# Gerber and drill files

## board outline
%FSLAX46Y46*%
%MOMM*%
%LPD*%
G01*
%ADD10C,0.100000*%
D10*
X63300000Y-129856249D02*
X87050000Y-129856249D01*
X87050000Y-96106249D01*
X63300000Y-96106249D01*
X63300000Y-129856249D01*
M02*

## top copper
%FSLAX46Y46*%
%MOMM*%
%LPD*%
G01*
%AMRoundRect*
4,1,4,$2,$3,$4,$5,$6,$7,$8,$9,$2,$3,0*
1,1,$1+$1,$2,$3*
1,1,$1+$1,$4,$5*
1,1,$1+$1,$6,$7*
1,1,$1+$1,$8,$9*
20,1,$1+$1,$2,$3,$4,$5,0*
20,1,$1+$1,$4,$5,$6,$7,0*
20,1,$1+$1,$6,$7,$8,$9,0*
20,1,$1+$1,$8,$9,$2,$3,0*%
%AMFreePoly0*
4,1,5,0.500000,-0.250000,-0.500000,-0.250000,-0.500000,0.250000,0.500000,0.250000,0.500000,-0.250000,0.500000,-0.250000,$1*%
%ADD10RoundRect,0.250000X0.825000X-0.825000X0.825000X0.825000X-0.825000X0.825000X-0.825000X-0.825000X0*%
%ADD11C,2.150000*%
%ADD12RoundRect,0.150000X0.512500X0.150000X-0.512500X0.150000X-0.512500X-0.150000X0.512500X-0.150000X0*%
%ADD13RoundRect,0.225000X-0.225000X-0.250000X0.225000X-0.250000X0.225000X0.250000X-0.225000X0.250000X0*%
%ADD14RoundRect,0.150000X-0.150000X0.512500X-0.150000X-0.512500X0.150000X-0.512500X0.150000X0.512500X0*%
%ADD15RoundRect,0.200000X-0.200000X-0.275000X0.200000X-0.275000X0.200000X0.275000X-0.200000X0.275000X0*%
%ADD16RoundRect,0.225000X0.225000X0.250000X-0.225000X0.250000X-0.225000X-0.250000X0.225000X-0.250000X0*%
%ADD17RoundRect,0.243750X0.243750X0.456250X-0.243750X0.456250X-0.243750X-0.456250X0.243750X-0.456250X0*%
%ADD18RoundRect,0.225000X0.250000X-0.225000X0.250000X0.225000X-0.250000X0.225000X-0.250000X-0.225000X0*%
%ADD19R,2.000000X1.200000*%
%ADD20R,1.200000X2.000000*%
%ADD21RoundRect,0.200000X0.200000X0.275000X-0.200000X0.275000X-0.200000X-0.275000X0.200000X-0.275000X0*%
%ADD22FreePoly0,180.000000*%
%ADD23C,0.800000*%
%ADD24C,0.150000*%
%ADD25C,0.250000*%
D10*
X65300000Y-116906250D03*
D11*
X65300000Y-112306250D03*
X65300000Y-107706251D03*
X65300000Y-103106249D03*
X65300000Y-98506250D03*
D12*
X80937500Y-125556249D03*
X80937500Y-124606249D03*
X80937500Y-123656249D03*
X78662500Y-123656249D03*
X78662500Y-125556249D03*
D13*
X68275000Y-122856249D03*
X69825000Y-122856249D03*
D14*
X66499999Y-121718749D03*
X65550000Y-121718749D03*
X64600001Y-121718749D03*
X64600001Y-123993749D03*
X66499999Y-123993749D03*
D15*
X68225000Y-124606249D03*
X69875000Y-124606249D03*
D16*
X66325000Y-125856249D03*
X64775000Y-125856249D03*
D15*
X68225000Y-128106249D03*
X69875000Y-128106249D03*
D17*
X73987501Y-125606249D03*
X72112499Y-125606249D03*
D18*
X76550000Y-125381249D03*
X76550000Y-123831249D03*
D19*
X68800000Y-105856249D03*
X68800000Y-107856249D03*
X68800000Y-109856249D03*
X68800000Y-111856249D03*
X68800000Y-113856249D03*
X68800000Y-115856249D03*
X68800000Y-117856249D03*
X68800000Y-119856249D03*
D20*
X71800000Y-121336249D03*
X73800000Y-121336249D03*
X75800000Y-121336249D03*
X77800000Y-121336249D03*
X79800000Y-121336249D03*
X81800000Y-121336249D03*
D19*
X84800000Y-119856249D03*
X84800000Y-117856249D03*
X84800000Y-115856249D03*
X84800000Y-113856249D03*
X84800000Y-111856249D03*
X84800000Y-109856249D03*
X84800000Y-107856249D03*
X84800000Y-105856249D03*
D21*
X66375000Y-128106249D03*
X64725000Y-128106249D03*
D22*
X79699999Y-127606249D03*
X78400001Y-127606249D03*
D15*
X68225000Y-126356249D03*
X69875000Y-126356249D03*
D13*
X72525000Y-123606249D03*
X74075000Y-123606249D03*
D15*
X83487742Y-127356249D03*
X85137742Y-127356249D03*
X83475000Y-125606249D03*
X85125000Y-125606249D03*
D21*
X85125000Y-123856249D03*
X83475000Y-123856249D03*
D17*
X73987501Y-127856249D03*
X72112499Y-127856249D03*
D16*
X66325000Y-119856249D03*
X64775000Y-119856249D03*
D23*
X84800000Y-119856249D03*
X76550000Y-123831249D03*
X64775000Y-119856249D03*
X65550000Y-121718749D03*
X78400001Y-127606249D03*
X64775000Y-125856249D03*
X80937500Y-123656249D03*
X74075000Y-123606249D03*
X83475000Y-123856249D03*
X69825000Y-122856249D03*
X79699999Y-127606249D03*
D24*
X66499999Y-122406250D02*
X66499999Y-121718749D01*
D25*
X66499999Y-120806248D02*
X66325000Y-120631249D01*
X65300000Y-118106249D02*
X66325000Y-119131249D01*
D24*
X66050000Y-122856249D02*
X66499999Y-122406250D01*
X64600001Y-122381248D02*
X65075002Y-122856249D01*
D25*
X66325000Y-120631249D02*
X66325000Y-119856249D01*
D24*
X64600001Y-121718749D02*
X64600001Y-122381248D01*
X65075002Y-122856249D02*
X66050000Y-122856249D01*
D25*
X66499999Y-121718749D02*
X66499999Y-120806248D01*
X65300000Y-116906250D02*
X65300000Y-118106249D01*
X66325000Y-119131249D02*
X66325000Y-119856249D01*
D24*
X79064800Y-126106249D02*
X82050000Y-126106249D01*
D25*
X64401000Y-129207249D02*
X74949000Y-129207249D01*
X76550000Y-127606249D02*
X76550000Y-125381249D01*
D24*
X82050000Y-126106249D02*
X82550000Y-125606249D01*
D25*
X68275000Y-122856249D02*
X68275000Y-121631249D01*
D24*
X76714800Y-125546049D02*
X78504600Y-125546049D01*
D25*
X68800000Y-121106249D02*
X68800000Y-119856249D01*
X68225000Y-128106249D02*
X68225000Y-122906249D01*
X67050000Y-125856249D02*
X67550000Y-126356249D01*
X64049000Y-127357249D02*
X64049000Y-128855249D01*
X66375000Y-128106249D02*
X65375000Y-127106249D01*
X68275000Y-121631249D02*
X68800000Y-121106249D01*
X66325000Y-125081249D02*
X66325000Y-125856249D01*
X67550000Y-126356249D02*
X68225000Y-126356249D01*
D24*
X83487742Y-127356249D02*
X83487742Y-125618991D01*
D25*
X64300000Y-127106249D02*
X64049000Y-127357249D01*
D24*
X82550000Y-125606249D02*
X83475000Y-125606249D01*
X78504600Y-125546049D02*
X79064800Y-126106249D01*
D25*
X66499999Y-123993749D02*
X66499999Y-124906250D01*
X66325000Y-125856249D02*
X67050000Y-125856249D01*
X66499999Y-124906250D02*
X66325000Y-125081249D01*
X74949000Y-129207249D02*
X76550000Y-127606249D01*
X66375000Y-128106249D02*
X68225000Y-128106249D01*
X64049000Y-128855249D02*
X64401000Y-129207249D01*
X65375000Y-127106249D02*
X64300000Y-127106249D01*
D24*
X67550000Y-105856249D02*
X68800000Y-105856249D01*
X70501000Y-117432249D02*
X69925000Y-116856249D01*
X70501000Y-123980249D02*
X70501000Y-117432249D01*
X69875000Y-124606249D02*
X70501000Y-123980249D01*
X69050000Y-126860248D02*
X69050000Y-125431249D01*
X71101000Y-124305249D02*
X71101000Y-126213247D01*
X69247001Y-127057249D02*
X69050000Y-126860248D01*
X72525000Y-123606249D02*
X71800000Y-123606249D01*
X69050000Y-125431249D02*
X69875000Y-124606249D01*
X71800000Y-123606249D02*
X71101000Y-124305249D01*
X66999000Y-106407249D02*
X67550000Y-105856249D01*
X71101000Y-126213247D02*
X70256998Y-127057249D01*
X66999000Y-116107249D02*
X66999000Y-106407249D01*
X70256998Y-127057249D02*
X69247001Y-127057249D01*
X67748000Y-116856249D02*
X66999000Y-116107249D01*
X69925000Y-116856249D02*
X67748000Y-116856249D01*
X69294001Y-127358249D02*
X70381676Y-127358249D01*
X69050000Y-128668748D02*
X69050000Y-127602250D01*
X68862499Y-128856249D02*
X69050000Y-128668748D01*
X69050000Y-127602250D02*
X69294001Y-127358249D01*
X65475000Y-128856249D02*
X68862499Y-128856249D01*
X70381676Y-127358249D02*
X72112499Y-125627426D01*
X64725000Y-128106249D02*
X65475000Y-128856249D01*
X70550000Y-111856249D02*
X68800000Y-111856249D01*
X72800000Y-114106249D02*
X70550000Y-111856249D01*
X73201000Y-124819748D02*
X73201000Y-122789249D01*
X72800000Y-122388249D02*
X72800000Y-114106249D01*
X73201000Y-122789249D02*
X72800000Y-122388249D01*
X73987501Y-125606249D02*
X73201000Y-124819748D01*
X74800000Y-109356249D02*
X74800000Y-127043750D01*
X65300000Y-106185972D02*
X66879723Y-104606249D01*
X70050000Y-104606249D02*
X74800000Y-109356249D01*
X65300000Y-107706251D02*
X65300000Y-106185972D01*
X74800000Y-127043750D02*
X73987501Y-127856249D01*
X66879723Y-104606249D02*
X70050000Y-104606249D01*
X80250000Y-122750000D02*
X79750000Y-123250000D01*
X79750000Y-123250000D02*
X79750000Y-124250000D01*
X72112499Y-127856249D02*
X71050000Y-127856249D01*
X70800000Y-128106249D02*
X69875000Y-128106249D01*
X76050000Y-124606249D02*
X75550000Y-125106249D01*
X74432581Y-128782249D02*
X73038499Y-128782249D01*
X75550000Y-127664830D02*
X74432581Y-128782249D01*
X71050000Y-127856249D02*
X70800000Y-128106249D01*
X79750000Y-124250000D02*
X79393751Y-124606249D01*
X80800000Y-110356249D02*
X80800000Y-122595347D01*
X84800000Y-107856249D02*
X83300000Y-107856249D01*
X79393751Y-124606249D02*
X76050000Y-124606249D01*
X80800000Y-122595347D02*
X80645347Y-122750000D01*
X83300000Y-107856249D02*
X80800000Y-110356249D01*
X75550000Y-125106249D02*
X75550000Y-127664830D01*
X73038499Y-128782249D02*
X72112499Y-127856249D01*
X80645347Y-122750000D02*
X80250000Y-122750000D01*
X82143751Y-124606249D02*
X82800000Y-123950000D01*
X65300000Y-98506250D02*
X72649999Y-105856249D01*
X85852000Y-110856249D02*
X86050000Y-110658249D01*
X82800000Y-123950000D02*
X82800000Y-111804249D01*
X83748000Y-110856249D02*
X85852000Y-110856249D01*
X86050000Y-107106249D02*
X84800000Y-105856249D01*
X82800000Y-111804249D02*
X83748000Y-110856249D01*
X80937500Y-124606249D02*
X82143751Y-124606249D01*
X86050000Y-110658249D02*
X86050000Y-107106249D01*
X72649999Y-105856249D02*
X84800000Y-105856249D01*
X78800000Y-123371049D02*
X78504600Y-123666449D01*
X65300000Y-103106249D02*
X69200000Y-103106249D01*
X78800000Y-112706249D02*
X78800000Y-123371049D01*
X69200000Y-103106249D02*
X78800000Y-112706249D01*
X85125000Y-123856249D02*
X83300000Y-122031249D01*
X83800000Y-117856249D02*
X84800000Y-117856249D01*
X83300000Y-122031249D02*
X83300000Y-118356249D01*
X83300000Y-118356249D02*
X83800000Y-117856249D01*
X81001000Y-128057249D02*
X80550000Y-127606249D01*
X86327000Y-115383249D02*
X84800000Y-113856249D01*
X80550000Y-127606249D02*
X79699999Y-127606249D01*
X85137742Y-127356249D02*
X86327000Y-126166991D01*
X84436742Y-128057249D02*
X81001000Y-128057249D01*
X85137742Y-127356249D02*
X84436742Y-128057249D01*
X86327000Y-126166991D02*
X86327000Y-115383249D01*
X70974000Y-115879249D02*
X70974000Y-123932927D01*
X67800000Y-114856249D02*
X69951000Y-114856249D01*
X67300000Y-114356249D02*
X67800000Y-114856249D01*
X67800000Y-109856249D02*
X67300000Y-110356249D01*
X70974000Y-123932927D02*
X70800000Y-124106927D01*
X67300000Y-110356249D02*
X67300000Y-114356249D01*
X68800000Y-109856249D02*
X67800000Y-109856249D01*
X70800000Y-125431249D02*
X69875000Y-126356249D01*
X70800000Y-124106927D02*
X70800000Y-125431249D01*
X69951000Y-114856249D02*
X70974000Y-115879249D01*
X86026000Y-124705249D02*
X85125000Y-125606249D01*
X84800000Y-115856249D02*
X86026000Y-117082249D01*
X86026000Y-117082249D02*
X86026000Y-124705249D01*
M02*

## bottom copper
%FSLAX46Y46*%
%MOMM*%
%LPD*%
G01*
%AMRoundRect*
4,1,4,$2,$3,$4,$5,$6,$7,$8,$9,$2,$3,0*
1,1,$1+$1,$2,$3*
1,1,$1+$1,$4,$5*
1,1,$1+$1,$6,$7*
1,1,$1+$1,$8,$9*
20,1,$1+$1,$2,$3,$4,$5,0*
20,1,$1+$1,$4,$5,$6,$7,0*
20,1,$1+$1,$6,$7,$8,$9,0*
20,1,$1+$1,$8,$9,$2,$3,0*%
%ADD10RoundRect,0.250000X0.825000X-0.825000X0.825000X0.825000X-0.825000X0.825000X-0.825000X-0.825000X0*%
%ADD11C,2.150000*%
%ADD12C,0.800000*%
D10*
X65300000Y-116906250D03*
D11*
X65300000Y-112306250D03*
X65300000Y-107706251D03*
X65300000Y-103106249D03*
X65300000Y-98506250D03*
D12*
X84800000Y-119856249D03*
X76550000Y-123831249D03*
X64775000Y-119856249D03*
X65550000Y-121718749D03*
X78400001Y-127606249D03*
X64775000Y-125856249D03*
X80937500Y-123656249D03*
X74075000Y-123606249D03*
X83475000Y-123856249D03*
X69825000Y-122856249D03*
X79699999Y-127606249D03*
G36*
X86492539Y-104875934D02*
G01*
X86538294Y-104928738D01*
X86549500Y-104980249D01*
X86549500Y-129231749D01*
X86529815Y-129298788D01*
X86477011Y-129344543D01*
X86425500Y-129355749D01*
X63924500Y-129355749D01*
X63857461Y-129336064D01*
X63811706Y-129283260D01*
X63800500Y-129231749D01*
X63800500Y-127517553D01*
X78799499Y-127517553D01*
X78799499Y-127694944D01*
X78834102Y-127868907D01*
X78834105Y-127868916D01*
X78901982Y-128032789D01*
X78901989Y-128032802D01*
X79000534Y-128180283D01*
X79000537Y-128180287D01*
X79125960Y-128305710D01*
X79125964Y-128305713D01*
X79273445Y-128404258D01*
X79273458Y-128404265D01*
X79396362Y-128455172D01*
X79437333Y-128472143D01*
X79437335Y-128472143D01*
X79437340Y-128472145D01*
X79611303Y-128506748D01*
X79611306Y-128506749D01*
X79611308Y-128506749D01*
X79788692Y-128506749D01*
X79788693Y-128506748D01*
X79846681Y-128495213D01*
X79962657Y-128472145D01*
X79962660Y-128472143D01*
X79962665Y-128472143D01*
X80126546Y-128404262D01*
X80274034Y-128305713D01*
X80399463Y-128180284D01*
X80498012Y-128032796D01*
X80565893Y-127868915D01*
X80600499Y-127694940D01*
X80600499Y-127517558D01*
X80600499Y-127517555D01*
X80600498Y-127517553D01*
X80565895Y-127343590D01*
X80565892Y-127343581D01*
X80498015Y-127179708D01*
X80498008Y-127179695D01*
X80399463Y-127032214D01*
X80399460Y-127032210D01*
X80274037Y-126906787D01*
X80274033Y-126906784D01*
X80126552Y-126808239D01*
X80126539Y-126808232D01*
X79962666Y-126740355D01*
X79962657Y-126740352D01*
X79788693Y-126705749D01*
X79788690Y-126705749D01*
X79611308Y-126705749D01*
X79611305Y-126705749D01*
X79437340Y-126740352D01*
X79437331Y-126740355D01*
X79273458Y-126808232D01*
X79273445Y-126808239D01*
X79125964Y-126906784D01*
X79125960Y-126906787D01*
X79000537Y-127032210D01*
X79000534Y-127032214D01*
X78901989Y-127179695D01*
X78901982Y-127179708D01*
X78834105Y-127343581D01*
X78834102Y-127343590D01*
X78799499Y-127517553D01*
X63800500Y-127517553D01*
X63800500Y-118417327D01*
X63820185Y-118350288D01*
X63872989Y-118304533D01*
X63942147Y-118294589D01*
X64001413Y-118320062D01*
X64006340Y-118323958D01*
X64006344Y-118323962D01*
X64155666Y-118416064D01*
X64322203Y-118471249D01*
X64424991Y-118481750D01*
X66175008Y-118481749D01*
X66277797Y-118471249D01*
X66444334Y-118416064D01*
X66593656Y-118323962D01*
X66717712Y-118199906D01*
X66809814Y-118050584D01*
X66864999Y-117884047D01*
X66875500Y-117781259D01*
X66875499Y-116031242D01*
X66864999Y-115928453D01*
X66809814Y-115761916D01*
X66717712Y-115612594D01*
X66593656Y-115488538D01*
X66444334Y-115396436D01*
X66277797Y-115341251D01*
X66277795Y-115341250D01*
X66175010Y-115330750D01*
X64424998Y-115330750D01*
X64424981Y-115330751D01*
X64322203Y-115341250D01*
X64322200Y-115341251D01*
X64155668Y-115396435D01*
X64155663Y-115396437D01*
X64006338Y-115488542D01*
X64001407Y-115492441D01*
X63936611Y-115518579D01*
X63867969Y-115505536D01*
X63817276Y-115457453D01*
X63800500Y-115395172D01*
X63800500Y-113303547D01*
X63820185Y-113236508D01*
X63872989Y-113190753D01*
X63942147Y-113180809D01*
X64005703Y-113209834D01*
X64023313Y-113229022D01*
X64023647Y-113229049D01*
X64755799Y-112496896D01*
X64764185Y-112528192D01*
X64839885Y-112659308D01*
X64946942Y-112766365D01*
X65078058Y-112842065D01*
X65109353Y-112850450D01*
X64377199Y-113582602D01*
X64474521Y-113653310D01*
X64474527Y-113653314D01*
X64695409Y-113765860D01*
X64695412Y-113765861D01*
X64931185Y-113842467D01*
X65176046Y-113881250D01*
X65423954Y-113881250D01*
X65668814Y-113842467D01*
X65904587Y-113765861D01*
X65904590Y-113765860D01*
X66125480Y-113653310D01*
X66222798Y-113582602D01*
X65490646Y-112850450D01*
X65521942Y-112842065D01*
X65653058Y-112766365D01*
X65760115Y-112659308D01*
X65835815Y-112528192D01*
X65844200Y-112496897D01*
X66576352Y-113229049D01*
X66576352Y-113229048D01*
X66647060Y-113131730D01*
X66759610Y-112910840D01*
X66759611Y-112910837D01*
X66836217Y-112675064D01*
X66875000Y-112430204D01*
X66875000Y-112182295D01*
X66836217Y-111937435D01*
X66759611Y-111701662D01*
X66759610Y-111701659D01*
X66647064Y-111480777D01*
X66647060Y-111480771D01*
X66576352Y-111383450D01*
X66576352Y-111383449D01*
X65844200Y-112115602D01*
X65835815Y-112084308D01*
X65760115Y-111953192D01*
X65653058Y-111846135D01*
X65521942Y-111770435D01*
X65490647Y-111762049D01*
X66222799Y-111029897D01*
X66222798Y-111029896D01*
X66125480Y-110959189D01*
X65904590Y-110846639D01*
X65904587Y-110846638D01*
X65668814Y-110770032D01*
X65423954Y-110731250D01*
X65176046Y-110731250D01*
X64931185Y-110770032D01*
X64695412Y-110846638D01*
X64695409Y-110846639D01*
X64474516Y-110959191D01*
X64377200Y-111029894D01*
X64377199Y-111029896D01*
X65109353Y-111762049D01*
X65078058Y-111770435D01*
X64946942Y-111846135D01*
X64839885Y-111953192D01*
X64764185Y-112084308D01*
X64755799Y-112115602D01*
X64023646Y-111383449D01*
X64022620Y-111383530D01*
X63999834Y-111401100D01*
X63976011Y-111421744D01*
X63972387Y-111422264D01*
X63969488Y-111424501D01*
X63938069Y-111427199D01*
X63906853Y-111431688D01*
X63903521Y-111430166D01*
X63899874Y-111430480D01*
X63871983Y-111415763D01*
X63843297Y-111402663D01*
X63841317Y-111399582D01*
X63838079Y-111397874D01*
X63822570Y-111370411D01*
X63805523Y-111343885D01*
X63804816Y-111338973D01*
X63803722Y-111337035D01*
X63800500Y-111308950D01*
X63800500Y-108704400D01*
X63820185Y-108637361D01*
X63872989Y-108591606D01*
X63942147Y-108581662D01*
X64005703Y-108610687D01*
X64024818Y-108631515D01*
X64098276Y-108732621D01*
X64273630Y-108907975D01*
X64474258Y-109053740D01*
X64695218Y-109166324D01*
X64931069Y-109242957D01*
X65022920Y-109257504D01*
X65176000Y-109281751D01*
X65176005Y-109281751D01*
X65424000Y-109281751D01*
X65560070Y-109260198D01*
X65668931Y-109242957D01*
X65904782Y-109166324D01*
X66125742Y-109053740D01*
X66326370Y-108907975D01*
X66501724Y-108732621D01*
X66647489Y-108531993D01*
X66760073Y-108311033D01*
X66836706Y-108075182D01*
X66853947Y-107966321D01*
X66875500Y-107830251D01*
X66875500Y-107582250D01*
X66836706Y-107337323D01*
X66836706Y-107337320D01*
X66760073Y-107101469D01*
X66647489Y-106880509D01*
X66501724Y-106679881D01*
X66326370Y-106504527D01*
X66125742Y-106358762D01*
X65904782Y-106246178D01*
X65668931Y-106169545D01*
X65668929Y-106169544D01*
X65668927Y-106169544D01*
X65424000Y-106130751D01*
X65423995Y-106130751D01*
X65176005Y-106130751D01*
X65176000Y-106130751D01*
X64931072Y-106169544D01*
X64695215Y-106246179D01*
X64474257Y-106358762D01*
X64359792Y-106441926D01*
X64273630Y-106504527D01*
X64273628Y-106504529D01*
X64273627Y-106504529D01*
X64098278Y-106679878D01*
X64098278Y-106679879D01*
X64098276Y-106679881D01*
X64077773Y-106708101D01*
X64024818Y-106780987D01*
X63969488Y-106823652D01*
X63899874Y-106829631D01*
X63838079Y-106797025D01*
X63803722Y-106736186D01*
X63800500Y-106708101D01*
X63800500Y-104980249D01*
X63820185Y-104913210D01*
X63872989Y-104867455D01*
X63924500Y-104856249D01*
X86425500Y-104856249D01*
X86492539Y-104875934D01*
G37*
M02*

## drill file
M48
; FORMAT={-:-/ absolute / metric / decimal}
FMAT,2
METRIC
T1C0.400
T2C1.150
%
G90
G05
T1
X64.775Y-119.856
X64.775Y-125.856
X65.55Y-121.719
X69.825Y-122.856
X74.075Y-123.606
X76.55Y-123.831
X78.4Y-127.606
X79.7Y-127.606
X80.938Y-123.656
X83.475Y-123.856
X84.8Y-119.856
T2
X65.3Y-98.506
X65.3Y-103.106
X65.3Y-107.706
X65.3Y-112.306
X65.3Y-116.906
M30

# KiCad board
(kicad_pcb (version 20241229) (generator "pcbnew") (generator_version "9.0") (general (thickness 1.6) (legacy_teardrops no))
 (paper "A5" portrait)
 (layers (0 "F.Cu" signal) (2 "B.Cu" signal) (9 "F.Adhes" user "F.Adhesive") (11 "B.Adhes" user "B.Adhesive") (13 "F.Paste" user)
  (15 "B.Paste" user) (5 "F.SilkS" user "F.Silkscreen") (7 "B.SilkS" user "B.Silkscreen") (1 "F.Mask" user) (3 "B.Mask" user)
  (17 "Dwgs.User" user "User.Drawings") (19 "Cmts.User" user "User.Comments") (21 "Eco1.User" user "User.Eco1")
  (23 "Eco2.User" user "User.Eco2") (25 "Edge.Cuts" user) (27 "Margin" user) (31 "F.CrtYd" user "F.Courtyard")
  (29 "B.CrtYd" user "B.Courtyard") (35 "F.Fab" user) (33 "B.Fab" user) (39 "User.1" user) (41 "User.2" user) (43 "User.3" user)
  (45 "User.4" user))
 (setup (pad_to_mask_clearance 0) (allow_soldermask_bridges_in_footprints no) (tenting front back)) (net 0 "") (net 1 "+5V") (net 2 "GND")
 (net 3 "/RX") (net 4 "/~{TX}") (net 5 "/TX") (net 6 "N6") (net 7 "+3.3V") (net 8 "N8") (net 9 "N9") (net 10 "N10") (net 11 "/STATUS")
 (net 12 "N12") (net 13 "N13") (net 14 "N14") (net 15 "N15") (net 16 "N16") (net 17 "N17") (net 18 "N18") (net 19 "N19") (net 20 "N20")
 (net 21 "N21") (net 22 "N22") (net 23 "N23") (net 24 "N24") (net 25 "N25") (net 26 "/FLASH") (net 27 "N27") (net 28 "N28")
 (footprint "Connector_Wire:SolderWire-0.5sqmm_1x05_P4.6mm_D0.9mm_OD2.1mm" (layer "F.Cu") (at 65.3 116.90625 90)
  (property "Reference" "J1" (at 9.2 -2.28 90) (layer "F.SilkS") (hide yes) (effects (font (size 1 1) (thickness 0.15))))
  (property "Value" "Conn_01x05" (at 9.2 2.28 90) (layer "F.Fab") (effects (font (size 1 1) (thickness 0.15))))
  (pad "1" thru_hole roundrect (at 0 0 90) (size 2.15 2.15) (drill 1.15) (layers "*.Cu" "*.Mask") (remove_unused_layers no)
   (roundrect_rratio 0.116279) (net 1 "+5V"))
  (pad "2" thru_hole circle (at 4.6 0 90) (size 2.15 2.15) (drill 1.15) (layers "*.Cu" "*.Mask") (remove_unused_layers no) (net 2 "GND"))
  (pad "3" thru_hole circle (at 9.199999 0 90) (size 2.15 2.15) (drill 1.15) (layers "*.Cu" "*.Mask") (remove_unused_layers no)
   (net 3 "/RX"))
  (pad "4" thru_hole circle (at 13.800001 0 90) (size 2.15 2.15) (drill 1.15) (layers "*.Cu" "*.Mask") (remove_unused_layers no)
   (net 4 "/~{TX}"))
  (pad "5" thru_hole circle (at 18.4 0 90) (size 2.15 2.15) (drill 1.15) (layers "*.Cu" "*.Mask") (remove_unused_layers no) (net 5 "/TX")))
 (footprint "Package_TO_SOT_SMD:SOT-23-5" (layer "F.Cu") (at 79.8 124.606249 180)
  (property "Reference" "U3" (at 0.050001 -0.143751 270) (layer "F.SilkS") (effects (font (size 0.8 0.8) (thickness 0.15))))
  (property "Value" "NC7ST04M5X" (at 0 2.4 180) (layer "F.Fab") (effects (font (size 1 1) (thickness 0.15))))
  (pad "1" smd roundrect (at -1.1375 -0.95 180) (size 1.325 0.6) (layers "F.Cu" "F.Mask" "F.Paste") (roundrect_rratio 0.25) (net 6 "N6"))
  (pad "2" smd roundrect (at -1.1375 0 180) (size 1.325 0.6) (layers "F.Cu" "F.Mask" "F.Paste") (roundrect_rratio 0.25) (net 5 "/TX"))
  (pad "3" smd roundrect (at -1.1375 0.95 180) (size 1.325 0.6) (layers "F.Cu" "F.Mask" "F.Paste") (roundrect_rratio 0.25) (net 2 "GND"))
  (pad "4" smd roundrect (at 1.1375 0.95 180) (size 1.325 0.6) (layers "F.Cu" "F.Mask" "F.Paste") (roundrect_rratio 0.25) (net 4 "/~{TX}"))
  (pad "5" smd roundrect (at 1.1375 -0.95 180) (size 1.325 0.6) (layers "F.Cu" "F.Mask" "F.Paste") (roundrect_rratio 0.25) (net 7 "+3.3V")))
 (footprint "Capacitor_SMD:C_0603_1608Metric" (layer "F.Cu") (at 69.05 122.856249)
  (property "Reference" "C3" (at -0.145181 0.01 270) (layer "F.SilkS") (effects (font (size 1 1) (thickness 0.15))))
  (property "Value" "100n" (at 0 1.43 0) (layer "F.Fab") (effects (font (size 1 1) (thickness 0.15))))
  (pad "1" smd roundrect (at -0.775 0) (size 0.9 0.95) (layers "F.Cu" "F.Mask" "F.Paste") (roundrect_rratio 0.25) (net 7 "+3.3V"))
  (pad "2" smd roundrect (at 0.775 0) (size 0.9 0.95) (layers "F.Cu" "F.Mask" "F.Paste") (roundrect_rratio 0.25) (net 2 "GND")))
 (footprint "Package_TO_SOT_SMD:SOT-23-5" (layer "F.Cu") (at 65.55 122.856249 -90)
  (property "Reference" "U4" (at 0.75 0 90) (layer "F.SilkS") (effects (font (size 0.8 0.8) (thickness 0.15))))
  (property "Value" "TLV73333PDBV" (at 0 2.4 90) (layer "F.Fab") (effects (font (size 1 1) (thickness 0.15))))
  (pad "1" smd roundrect (at -1.1375 -0.949999 270) (size 1.325 0.6) (layers "F.Cu" "F.Mask" "F.Paste") (roundrect_rratio 0.25)
   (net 1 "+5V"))
  (pad "2" smd roundrect (at -1.1375 0 270) (size 1.325 0.6) (layers "F.Cu" "F.Mask" "F.Paste") (roundrect_rratio 0.25) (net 2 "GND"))
  (pad "3" smd roundrect (at -1.1375 0.949999 270) (size 1.325 0.6) (layers "F.Cu" "F.Mask" "F.Paste") (roundrect_rratio 0.25) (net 1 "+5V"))
  (pad "4" smd roundrect (at 1.1375 0.949999 270) (size 1.325 0.6) (layers "F.Cu" "F.Mask" "F.Paste") (roundrect_rratio 0.25) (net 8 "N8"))
  (pad "5" smd roundrect (at 1.1375 -0.949999 270) (size 1.325 0.6) (layers "F.Cu" "F.Mask" "F.Paste") (roundrect_rratio 0.25)
   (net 7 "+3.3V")))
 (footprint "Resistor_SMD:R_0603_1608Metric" (layer "F.Cu") (at 69.05 124.606249)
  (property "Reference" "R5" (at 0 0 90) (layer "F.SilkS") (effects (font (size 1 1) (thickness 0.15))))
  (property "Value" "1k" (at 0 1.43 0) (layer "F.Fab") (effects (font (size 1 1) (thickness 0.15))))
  (pad "1" smd roundrect (at -0.825 0) (size 0.8 0.95) (layers "F.Cu" "F.Mask" "F.Paste") (roundrect_rratio 0.25) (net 7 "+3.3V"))
  (pad "2" smd roundrect (at 0.825 0) (size 0.8 0.95) (layers "F.Cu" "F.Mask" "F.Paste") (roundrect_rratio 0.25) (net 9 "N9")))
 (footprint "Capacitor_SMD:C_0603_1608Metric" (layer "F.Cu") (at 65.55 125.856249 180)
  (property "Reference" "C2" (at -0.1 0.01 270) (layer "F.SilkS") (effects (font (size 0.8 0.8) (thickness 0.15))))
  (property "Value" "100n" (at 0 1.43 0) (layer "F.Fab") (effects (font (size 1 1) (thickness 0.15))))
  (pad "1" smd roundrect (at -0.775 0 180) (size 0.9 0.95) (layers "F.Cu" "F.Mask" "F.Paste") (roundrect_rratio 0.25) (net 7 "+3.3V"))
  (pad "2" smd roundrect (at 0.775 0 180) (size 0.9 0.95) (layers "F.Cu" "F.Mask" "F.Paste") (roundrect_rratio 0.25) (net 2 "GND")))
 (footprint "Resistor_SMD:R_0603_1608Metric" (layer "F.Cu") (at 69.05 128.106249)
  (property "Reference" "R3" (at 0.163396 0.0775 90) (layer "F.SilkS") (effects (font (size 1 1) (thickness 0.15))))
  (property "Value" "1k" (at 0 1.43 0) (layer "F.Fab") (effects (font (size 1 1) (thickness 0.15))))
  (pad "1" smd roundrect (at -0.825 0) (size 0.8 0.95) (layers "F.Cu" "F.Mask" "F.Paste") (roundrect_rratio 0.25) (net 7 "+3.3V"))
  (pad "2" smd roundrect (at 0.825 0) (size 0.8 0.95) (layers "F.Cu" "F.Mask" "F.Paste") (roundrect_rratio 0.25) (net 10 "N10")))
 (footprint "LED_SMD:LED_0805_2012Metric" (layer "F.Cu") (at 73.05 125.606249 180)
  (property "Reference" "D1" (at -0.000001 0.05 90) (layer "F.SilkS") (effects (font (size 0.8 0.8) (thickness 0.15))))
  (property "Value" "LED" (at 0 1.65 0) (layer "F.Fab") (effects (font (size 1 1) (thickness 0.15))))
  (pad "1" smd roundrect (at -0.937501 0 180) (size 0.975 1.4) (layers "F.Cu" "F.Mask" "F.Paste") (roundrect_rratio 0.25) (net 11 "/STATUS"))
  (pad "2" smd roundrect (at 0.937501 0 180) (size 0.975 1.4) (layers "F.Cu" "F.Mask" "F.Paste") (roundrect_rratio 0.25) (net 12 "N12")))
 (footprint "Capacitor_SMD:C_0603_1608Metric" (layer "F.Cu") (at 76.55 124.606249 90)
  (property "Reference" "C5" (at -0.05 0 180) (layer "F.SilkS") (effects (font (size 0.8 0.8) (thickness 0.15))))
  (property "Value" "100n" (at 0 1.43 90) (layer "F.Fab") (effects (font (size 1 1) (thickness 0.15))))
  (pad "1" smd roundrect (at -0.775 0 90) (size 0.9 0.95) (layers "F.Cu" "F.Mask" "F.Paste") (roundrect_rratio 0.25) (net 7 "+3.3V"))
  (pad "2" smd roundrect (at 0.775 0 90) (size 0.9 0.95) (layers "F.Cu" "F.Mask" "F.Paste") (roundrect_rratio 0.25) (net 2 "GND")))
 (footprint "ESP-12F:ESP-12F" (layer "F.Cu") (at 76.8 109.336249)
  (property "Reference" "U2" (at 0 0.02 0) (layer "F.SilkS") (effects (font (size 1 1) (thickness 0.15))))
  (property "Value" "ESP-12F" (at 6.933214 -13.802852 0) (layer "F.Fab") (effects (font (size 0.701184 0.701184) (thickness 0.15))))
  (pad "1" smd rect (at -8 -3.48) (size 2 1.2) (layers "F.Cu" "F.Mask" "F.Paste") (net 9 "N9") (solder_mask_margin 0.102))
  (pad "2" smd rect (at -8 -1.48) (size 2 1.2) (layers "F.Cu" "F.Mask" "F.Paste") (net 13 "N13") (solder_mask_margin 0.102))
  (pad "3" smd rect (at -8 0.52) (size 2 1.2) (layers "F.Cu" "F.Mask" "F.Paste") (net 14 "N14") (solder_mask_margin 0.102))
  (pad "4" smd rect (at -8 2.52) (size 2 1.2) (layers "F.Cu" "F.Mask" "F.Paste") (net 11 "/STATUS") (solder_mask_margin 0.102))
  (pad "5" smd rect (at -8 4.52) (size 2 1.2) (layers "F.Cu" "F.Mask" "F.Paste") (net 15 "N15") (solder_mask_margin 0.102))
  (pad "6" smd rect (at -8 6.52) (size 2 1.2) (layers "F.Cu" "F.Mask" "F.Paste") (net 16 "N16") (solder_mask_margin 0.102))
  (pad "7" smd rect (at -8 8.52) (size 2 1.2) (layers "F.Cu" "F.Mask" "F.Paste") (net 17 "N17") (solder_mask_margin 0.102))
  (pad "8" smd rect (at -8 10.52) (size 2 1.2) (layers "F.Cu" "F.Mask" "F.Paste") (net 7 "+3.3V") (solder_mask_margin 0.102))
  (pad "9" smd rect (at -5 12) (size 1.2 2) (layers "F.Cu" "F.Mask" "F.Paste") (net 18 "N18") (solder_mask_margin 0.102))
  (pad "10" smd rect (at -3 12) (size 1.2 2) (layers "F.Cu" "F.Mask" "F.Paste") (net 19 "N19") (solder_mask_margin 0.102))
  (pad "11" smd rect (at -1 12) (size 1.2 2) (layers "F.Cu" "F.Mask" "F.Paste") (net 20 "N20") (solder_mask_margin 0.102))
  (pad "12" smd rect (at 1 12) (size 1.2 2) (layers "F.Cu" "F.Mask" "F.Paste") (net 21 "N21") (solder_mask_margin 0.102))
  (pad "13" smd rect (at 3 12) (size 1.2 2) (layers "F.Cu" "F.Mask" "F.Paste") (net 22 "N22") (solder_mask_margin 0.102))
  (pad "14" smd rect (at 5 12) (size 1.2 2) (layers "F.Cu" "F.Mask" "F.Paste") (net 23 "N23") (solder_mask_margin 0.102))
  (pad "15" smd rect (at 8 10.52) (size 2 1.2) (layers "F.Cu" "F.Mask" "F.Paste") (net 2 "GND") (solder_mask_margin 0.102))
  (pad "16" smd rect (at 8 8.52) (size 2 1.2) (layers "F.Cu" "F.Mask" "F.Paste") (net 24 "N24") (solder_mask_margin 0.102))
  (pad "17" smd rect (at 8 6.52) (size 2 1.2) (layers "F.Cu" "F.Mask" "F.Paste") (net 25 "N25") (solder_mask_margin 0.102))
  (pad "18" smd rect (at 8 4.52) (size 2 1.2) (layers "F.Cu" "F.Mask" "F.Paste") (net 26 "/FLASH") (solder_mask_margin 0.102))
  (pad "19" smd rect (at 8 2.52) (size 2 1.2) (layers "F.Cu" "F.Mask" "F.Paste") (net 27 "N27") (solder_mask_margin 0.102))
  (pad "20" smd rect (at 8 0.52) (size 2 1.2) (layers "F.Cu" "F.Mask" "F.Paste") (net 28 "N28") (solder_mask_margin 0.102))
  (pad "21" smd rect (at 8 -1.48) (size 2 1.2) (layers "F.Cu" "F.Mask" "F.Paste") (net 10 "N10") (solder_mask_margin 0.102))
  (pad "22" smd rect (at 8 -3.48) (size 2 1.2) (layers "F.Cu" "F.Mask" "F.Paste") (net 5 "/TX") (solder_mask_margin 0.102)))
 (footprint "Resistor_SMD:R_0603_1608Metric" (layer "F.Cu") (at 65.55 128.106249 180)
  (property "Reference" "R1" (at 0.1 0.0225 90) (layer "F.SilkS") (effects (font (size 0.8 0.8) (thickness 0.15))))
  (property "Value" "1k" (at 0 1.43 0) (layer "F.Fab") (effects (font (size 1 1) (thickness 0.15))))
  (pad "1" smd roundrect (at -0.825 0 180) (size 0.8 0.95) (layers "F.Cu" "F.Mask" "F.Paste") (roundrect_rratio 0.25) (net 7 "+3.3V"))
  (pad "2" smd roundrect (at 0.825 0 180) (size 0.8 0.95) (layers "F.Cu" "F.Mask" "F.Paste") (roundrect_rratio 0.25) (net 12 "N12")))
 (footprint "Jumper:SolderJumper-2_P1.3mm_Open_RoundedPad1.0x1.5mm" (layer "F.Cu") (at 79.05 127.606249 180)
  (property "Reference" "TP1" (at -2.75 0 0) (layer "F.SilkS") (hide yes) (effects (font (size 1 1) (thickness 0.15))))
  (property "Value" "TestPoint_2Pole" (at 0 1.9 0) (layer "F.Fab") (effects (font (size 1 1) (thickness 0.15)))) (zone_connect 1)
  (pad "1" smd custom (at -0.649999 0 180) (size 1 0.5) (layers "F.Cu" "F.Mask") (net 26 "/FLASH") (zone_connect 2)
   (thermal_bridge_angle 45) (options (clearance outline) (anchor rect)) (primitives))
  (pad "2" smd custom (at 0.649999 0 180) (size 1 0.5) (layers "F.Cu" "F.Mask") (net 2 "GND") (zone_connect 2) (thermal_bridge_angle 45)
   (options (clearance outline) (anchor rect)) (primitives)))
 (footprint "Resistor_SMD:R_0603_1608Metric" (layer "F.Cu") (at 69.05 126.356249)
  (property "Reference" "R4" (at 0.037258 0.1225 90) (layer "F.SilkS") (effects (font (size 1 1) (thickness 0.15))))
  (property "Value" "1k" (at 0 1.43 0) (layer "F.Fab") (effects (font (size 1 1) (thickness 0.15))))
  (pad "1" smd roundrect (at -0.825 0) (size 0.8 0.95) (layers "F.Cu" "F.Mask" "F.Paste") (roundrect_rratio 0.25) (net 7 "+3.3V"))
  (pad "2" smd roundrect (at 0.825 0) (size 0.8 0.95) (layers "F.Cu" "F.Mask" "F.Paste") (roundrect_rratio 0.25) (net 14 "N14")))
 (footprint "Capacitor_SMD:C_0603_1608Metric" (layer "F.Cu") (at 73.3 123.606249)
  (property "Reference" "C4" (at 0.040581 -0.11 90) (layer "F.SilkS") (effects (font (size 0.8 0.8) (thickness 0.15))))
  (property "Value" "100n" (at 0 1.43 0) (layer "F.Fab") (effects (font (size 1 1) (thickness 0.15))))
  (pad "1" smd roundrect (at -0.775 0) (size 0.9 0.95) (layers "F.Cu" "F.Mask" "F.Paste") (roundrect_rratio 0.25) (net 9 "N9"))
  (pad "2" smd roundrect (at 0.775 0) (size 0.9 0.95) (layers "F.Cu" "F.Mask" "F.Paste") (roundrect_rratio 0.25) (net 2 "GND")))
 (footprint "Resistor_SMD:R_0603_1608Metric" (layer "F.Cu") (at 84.312742 127.356249)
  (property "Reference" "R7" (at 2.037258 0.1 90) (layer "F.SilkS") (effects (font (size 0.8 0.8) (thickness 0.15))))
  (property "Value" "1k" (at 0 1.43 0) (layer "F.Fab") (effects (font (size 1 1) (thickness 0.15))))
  (pad "1" smd roundrect (at -0.825 0) (size 0.8 0.95) (layers "F.Cu" "F.Mask" "F.Paste") (roundrect_rratio 0.25) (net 7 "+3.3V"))
  (pad "2" smd roundrect (at 0.825 0) (size 0.8 0.95) (layers "F.Cu" "F.Mask" "F.Paste") (roundrect_rratio 0.25) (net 26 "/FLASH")))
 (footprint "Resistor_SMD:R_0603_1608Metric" (layer "F.Cu") (at 84.3 125.606249)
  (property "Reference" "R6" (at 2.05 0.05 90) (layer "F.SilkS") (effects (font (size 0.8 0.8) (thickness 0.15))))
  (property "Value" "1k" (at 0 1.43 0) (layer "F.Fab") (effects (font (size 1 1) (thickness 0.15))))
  (pad "1" smd roundrect (at -0.825 0) (size 0.8 0.95) (layers "F.Cu" "F.Mask" "F.Paste") (roundrect_rratio 0.25) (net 7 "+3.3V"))
  (pad "2" smd roundrect (at 0.825 0) (size 0.8 0.95) (layers "F.Cu" "F.Mask" "F.Paste") (roundrect_rratio 0.25) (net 25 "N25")))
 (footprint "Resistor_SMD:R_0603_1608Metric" (layer "F.Cu") (at 84.3 123.856249 180)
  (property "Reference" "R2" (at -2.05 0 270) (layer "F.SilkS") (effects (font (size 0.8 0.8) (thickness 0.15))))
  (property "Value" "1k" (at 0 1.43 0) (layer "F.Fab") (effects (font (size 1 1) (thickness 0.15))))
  (pad "1" smd roundrect (at -0.825 0 180) (size 0.8 0.95) (layers "F.Cu" "F.Mask" "F.Paste") (roundrect_rratio 0.25) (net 24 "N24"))
  (pad "2" smd roundrect (at 0.825 0 180) (size 0.8 0.95) (layers "F.Cu" "F.Mask" "F.Paste") (roundrect_rratio 0.25) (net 2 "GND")))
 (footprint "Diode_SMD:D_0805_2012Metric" (layer "F.Cu") (at 73.05 127.856249 180)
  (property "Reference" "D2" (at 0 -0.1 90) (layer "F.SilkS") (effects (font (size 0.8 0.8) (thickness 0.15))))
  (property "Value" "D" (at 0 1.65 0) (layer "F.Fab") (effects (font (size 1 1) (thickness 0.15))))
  (pad "1" smd roundrect (at -0.937501 0 180) (size 0.975 1.4) (layers "F.Cu" "F.Mask" "F.Paste") (roundrect_rratio 0.25) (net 3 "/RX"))
  (pad "2" smd roundrect (at 0.937501 0 180) (size 0.975 1.4) (layers "F.Cu" "F.Mask" "F.Paste") (roundrect_rratio 0.25) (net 10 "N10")))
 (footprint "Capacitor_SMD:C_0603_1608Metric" (layer "F.Cu") (at 65.55 119.856249 180)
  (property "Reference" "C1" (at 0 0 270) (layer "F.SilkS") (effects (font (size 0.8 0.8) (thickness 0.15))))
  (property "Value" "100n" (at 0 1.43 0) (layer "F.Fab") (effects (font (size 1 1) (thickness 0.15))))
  (pad "1" smd roundrect (at -0.775 0 180) (size 0.9 0.95) (layers "F.Cu" "F.Mask" "F.Paste") (roundrect_rratio 0.25) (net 1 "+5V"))
  (pad "2" smd roundrect (at 0.775 0 180) (size 0.9 0.95) (layers "F.Cu" "F.Mask" "F.Paste") (roundrect_rratio 0.25) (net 2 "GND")))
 (gr_poly
  (pts (xy 63.3 129.856249) (xy 87.05 129.856249) (xy 87.05 96.106249) (xy 63.3 96.106249)) (stroke (width 0.1) (type solid)) (fill no)
  (layer "Edge.Cuts"))
 (segment (start 66.499999 122.40625) (end 66.499999 121.718749) (width 0.15) (layer "F.Cu") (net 1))
 (segment (start 66.499999 120.806248) (end 66.325 120.631249) (width 0.25) (layer "F.Cu") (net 1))
 (segment (start 65.3 118.106249) (end 66.325 119.131249) (width 0.25) (layer "F.Cu") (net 1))
 (segment (start 66.05 122.856249) (end 66.499999 122.40625) (width 0.15) (layer "F.Cu") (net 1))
 (segment (start 64.600001 122.381248) (end 65.075002 122.856249) (width 0.15) (layer "F.Cu") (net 1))
 (segment (start 66.325 120.631249) (end 66.325 119.856249) (width 0.25) (layer "F.Cu") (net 1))
 (segment (start 64.600001 121.718749) (end 64.600001 122.381248) (width 0.15) (layer "F.Cu") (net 1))
 (segment (start 65.075002 122.856249) (end 66.05 122.856249) (width 0.15) (layer "F.Cu") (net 1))
 (segment (start 66.499999 121.718749) (end 66.499999 120.806248) (width 0.25) (layer "F.Cu") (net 1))
 (segment (start 65.3 116.90625) (end 65.3 118.106249) (width 0.25) (layer "F.Cu") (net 1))
 (segment (start 66.325 119.131249) (end 66.325 119.856249) (width 0.25) (layer "F.Cu") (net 1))
 (via (at 84.8 119.856249) (size 0.8) (drill 0.4) (layers "F.Cu" "B.Cu") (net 2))
 (via (at 76.55 123.831249) (size 0.8) (drill 0.4) (layers "F.Cu" "B.Cu") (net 2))
 (via (at 64.775 119.856249) (size 0.8) (drill 0.4) (layers "F.Cu" "B.Cu") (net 2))
 (via (at 65.55 121.718749) (size 0.8) (drill 0.4) (layers "F.Cu" "B.Cu") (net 2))
 (via (at 78.400001 127.606249) (size 0.8) (drill 0.4) (layers "F.Cu" "B.Cu") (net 2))
 (via (at 64.775 125.856249) (size 0.8) (drill 0.4) (layers "F.Cu" "B.Cu") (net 2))
 (via (at 80.9375 123.656249) (size 0.8) (drill 0.4) (layers "F.Cu" "B.Cu") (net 2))
 (via (at 74.075 123.606249) (size 0.8) (drill 0.4) (layers "F.Cu" "B.Cu") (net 2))
 (via (at 83.475 123.856249) (size 0.8) (drill 0.4) (layers "F.Cu" "B.Cu") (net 2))
 (via (at 69.825 122.856249) (size 0.8) (drill 0.4) (layers "F.Cu" "B.Cu") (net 2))
 (segment (start 79.0648 126.106249) (end 82.05 126.106249) (width 0.15) (layer "F.Cu") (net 7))
 (segment (start 64.401 129.207249) (end 74.949 129.207249) (width 0.25) (layer "F.Cu") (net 7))
 (segment (start 76.55 127.606249) (end 76.55 125.381249) (width 0.25) (layer "F.Cu") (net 7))
 (segment (start 82.05 126.106249) (end 82.55 125.606249) (width 0.15) (layer "F.Cu") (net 7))
 (segment (start 68.275 122.856249) (end 68.275 121.631249) (width 0.25) (layer "F.Cu") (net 7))
 (segment (start 76.7148 125.546049) (end 78.5046 125.546049) (width 0.15) (layer "F.Cu") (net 7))
 (segment (start 68.8 121.106249) (end 68.8 119.856249) (width 0.25) (layer "F.Cu") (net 7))
 (segment (start 68.225 128.106249) (end 68.225 122.906249) (width 0.25) (layer "F.Cu") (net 7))
 (segment (start 67.05 125.856249) (end 67.55 126.356249) (width 0.25) (layer "F.Cu") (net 7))
 (segment (start 64.049 127.357249) (end 64.049 128.855249) (width 0.25) (layer "F.Cu") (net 7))
 (segment (start 66.375 128.106249) (end 65.375 127.106249) (width 0.25) (layer "F.Cu") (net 7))
 (segment (start 68.275 121.631249) (end 68.8 121.106249) (width 0.25) (layer "F.Cu") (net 7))
 (segment (start 66.325 125.081249) (end 66.325 125.856249) (width 0.25) (layer "F.Cu") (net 7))
 (segment (start 67.55 126.356249) (end 68.225 126.356249) (width 0.25) (layer "F.Cu") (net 7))
 (segment (start 83.487742 127.356249) (end 83.487742 125.618991) (width 0.15) (layer "F.Cu") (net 7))
 (segment (start 64.3 127.106249) (end 64.049 127.357249) (width 0.25) (layer "F.Cu") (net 7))
 (segment (start 82.55 125.606249) (end 83.475 125.606249) (width 0.15) (layer "F.Cu") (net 7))
 (segment (start 78.5046 125.546049) (end 79.0648 126.106249) (width 0.15) (layer "F.Cu") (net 7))
 (segment (start 66.499999 123.993749) (end 66.499999 124.90625) (width 0.25) (layer "F.Cu") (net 7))
 (segment (start 66.325 125.856249) (end 67.05 125.856249) (width 0.25) (layer "F.Cu") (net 7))
 (segment (start 66.499999 124.90625) (end 66.325 125.081249) (width 0.25) (layer "F.Cu") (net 7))
 (segment (start 74.949 129.207249) (end 76.55 127.606249) (width 0.25) (layer "F.Cu") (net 7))
 (segment (start 66.375 128.106249) (end 68.225 128.106249) (width 0.25) (layer "F.Cu") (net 7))
 (segment (start 64.049 128.855249) (end 64.401 129.207249) (width 0.25) (layer "F.Cu") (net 7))
 (segment (start 65.375 127.106249) (end 64.3 127.106249) (width 0.25) (layer "F.Cu") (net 7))
 (segment (start 67.55 105.856249) (end 68.8 105.856249) (width 0.15) (layer "F.Cu") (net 9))
 (segment (start 70.501 117.432249) (end 69.925 116.856249) (width 0.15) (layer "F.Cu") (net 9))
 (segment (start 70.501 123.980249) (end 70.501 117.432249) (width 0.15) (layer "F.Cu") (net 9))
 (segment (start 69.875 124.606249) (end 70.501 123.980249) (width 0.15) (layer "F.Cu") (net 9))
 (segment (start 69.05 126.860248) (end 69.05 125.431249) (width 0.15) (layer "F.Cu") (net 9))
 (segment (start 71.101 124.305249) (end 71.101 126.213247) (width 0.15) (layer "F.Cu") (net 9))
 (segment (start 69.247001 127.057249) (end 69.05 126.860248) (width 0.15) (layer "F.Cu") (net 9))
 (segment (start 72.525 123.606249) (end 71.8 123.606249) (width 0.15) (layer "F.Cu") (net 9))
 (segment (start 69.05 125.431249) (end 69.875 124.606249) (width 0.15) (layer "F.Cu") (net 9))
 (segment (start 71.8 123.606249) (end 71.101 124.305249) (width 0.15) (layer "F.Cu") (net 9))
 (segment (start 66.999 106.407249) (end 67.55 105.856249) (width 0.15) (layer "F.Cu") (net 9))
 (segment (start 71.101 126.213247) (end 70.256998 127.057249) (width 0.15) (layer "F.Cu") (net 9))
 (segment (start 66.999 116.107249) (end 66.999 106.407249) (width 0.15) (layer "F.Cu") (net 9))
 (segment (start 70.256998 127.057249) (end 69.247001 127.057249) (width 0.15) (layer "F.Cu") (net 9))
 (segment (start 67.748 116.856249) (end 66.999 116.107249) (width 0.15) (layer "F.Cu") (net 9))
 (segment (start 69.925 116.856249) (end 67.748 116.856249) (width 0.15) (layer "F.Cu") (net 9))
 (segment (start 69.294001 127.358249) (end 70.381676 127.358249) (width 0.15) (layer "F.Cu") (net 12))
 (segment (start 69.05 128.668748) (end 69.05 127.60225) (width 0.15) (layer "F.Cu") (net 12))
 (segment (start 68.862499 128.856249) (end 69.05 128.668748) (width 0.15) (layer "F.Cu") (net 12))
 (segment (start 69.05 127.60225) (end 69.294001 127.358249) (width 0.15) (layer "F.Cu") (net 12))
 (segment (start 65.475 128.856249) (end 68.862499 128.856249) (width 0.15) (layer "F.Cu") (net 12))
 (segment (start 70.381676 127.358249) (end 72.112499 125.627426) (width 0.15) (layer "F.Cu") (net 12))
 (segment (start 64.725 128.106249) (end 65.475 128.856249) (width 0.15) (layer "F.Cu") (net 12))
 (segment (start 70.55 111.856249) (end 68.8 111.856249) (width 0.15) (layer "F.Cu") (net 11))
 (segment (start 72.8 114.106249) (end 70.55 111.856249) (width 0.15) (layer "F.Cu") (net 11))
 (segment (start 73.201 124.819748) (end 73.201 122.789249) (width 0.15) (layer "F.Cu") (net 11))
 (segment (start 72.8 122.388249) (end 72.8 114.106249) (width 0.15) (layer "F.Cu") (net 11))
 (segment (start 73.201 122.789249) (end 72.8 122.388249) (width 0.15) (layer "F.Cu") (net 11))
 (segment (start 73.987501 125.606249) (end 73.201 124.819748) (width 0.15) (layer "F.Cu") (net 11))
 (segment (start 74.8 109.356249) (end 74.8 127.04375) (width 0.15) (layer "F.Cu") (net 3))
 (segment (start 65.3 106.185972) (end 66.879723 104.606249) (width 0.15) (layer "F.Cu") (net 3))
 (segment (start 70.05 104.606249) (end 74.8 109.356249) (width 0.15) (layer "F.Cu") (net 3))
 (segment (start 65.3 107.706251) (end 65.3 106.185972) (width 0.15) (layer "F.Cu") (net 3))
 (segment (start 74.8 127.04375) (end 73.987501 127.856249) (width 0.15) (layer "F.Cu") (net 3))
 (segment (start 66.879723 104.606249) (end 70.05 104.606249) (width 0.15) (layer "F.Cu") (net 3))
 (segment (start 80.25 122.75) (end 79.75 123.25) (width 0.15) (layer "F.Cu") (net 10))
 (segment (start 79.75 123.25) (end 79.75 124.25) (width 0.15) (layer "F.Cu") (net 10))
 (segment (start 72.112499 127.856249) (end 71.05 127.856249) (width 0.15) (layer "F.Cu") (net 10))
 (segment (start 70.8 128.106249) (end 69.875 128.106249) (width 0.15) (layer "F.Cu") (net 10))
 (segment (start 76.05 124.606249) (end 75.55 125.106249) (width 0.15) (layer "F.Cu") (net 10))
 (segment (start 74.432581 128.782249) (end 73.038499 128.782249) (width 0.15) (layer "F.Cu") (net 10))
 (segment (start 75.55 127.66483) (end 74.432581 128.782249) (width 0.15) (layer "F.Cu") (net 10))
 (segment (start 71.05 127.856249) (end 70.8 128.106249) (width 0.15) (layer "F.Cu") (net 10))
 (segment (start 79.75 124.25) (end 79.393751 124.606249) (width 0.15) (layer "F.Cu") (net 10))
 (segment (start 80.8 110.356249) (end 80.8 122.595347) (width 0.15) (layer "F.Cu") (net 10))
 (segment (start 84.8 107.856249) (end 83.3 107.856249) (width 0.15) (layer "F.Cu") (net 10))
 (segment (start 79.393751 124.606249) (end 76.05 124.606249) (width 0.15) (layer "F.Cu") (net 10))
 (segment (start 80.8 122.595347) (end 80.645347 122.75) (width 0.15) (layer "F.Cu") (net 10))
 (segment (start 83.3 107.856249) (end 80.8 110.356249) (width 0.15) (layer "F.Cu") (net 10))
 (segment (start 75.55 125.106249) (end 75.55 127.66483) (width 0.15) (layer "F.Cu") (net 10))
 (segment (start 73.038499 128.782249) (end 72.112499 127.856249) (width 0.15) (layer "F.Cu") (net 10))
 (segment (start 80.645347 122.75) (end 80.25 122.75) (width 0.15) (layer "F.Cu") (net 10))
 (segment (start 82.143751 124.606249) (end 82.8 123.95) (width 0.15) (layer "F.Cu") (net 5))
 (segment (start 65.3 98.50625) (end 72.649999 105.856249) (width 0.15) (layer "F.Cu") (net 5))
 (segment (start 85.852 110.856249) (end 86.05 110.658249) (width 0.15) (layer "F.Cu") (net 5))
 (segment (start 82.8 123.95) (end 82.8 111.804249) (width 0.15) (layer "F.Cu") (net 5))
 (segment (start 83.748 110.856249) (end 85.852 110.856249) (width 0.15) (layer "F.Cu") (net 5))
 (segment (start 86.05 107.106249) (end 84.8 105.856249) (width 0.15) (layer "F.Cu") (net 5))
 (segment (start 82.8 111.804249) (end 83.748 110.856249) (width 0.15) (layer "F.Cu") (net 5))
 (segment (start 80.9375 124.606249) (end 82.143751 124.606249) (width 0.15) (layer "F.Cu") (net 5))
 (segment (start 86.05 110.658249) (end 86.05 107.106249) (width 0.15) (layer "F.Cu") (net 5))
 (segment (start 72.649999 105.856249) (end 84.8 105.856249) (width 0.15) (layer "F.Cu") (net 5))
 (segment (start 78.8 123.371049) (end 78.5046 123.666449) (width 0.15) (layer "F.Cu") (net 4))
 (segment (start 65.3 103.106249) (end 69.2 103.106249) (width 0.15) (layer "F.Cu") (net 4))
 (segment (start 78.8 112.706249) (end 78.8 123.371049) (width 0.15) (layer "F.Cu") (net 4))
 (segment (start 69.2 103.106249) (end 78.8 112.706249) (width 0.15) (layer "F.Cu") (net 4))
 (segment (start 85.125 123.856249) (end 83.3 122.031249) (width 0.15) (layer "F.Cu") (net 24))
 (segment (start 83.8 117.856249) (end 84.8 117.856249) (width 0.15) (layer "F.Cu") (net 24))
 (segment (start 83.3 122.031249) (end 83.3 118.356249) (width 0.15) (layer "F.Cu") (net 24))
 (segment (start 83.3 118.356249) (end 83.8 117.856249) (width 0.15) (layer "F.Cu") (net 24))
 (segment (start 81.001 128.057249) (end 80.55 127.606249) (width 0.15) (layer "F.Cu") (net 26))
 (segment (start 86.327 115.383249) (end 84.8 113.856249) (width 0.15) (layer "F.Cu") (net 26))
 (segment (start 80.55 127.606249) (end 79.699999 127.606249) (width 0.15) (layer "F.Cu") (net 26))
 (segment (start 85.137742 127.356249) (end 86.327 126.166991) (width 0.15) (layer "F.Cu") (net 26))
 (segment (start 84.436742 128.057249) (end 81.001 128.057249) (width 0.15) (layer "F.Cu") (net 26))
 (segment (start 85.137742 127.356249) (end 84.436742 128.057249) (width 0.15) (layer "F.Cu") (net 26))
 (segment (start 86.327 126.166991) (end 86.327 115.383249) (width 0.15) (layer "F.Cu") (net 26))
 (via (at 79.699999 127.606249) (size 0.8) (drill 0.4) (layers "F.Cu" "B.Cu") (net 26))
 (segment (start 70.974 115.879249) (end 70.974 123.932927) (width 0.15) (layer "F.Cu") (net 14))
 (segment (start 67.8 114.856249) (end 69.951 114.856249) (width 0.15) (layer "F.Cu") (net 14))
 (segment (start 67.3 114.356249) (end 67.8 114.856249) (width 0.15) (layer "F.Cu") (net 14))
 (segment (start 67.8 109.856249) (end 67.3 110.356249) (width 0.15) (layer "F.Cu") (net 14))
 (segment (start 70.974 123.932927) (end 70.8 124.106927) (width 0.15) (layer "F.Cu") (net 14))
 (segment (start 67.3 110.356249) (end 67.3 114.356249) (width 0.15) (layer "F.Cu") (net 14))
 (segment (start 68.8 109.856249) (end 67.8 109.856249) (width 0.15) (layer "F.Cu") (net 14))
 (segment (start 70.8 125.431249) (end 69.875 126.356249) (width 0.15) (layer "F.Cu") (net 14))
 (segment (start 70.8 124.106927) (end 70.8 125.431249) (width 0.15) (layer "F.Cu") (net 14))
 (segment (start 69.951 114.856249) (end 70.974 115.879249) (width 0.15) (layer "F.Cu") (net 14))
 (segment (start 86.026 124.705249) (end 85.125 125.606249) (width 0.15) (layer "F.Cu") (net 25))
 (segment (start 84.8 115.856249) (end 86.026 117.082249) (width 0.15) (layer "F.Cu") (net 25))
 (segment (start 86.026 117.082249) (end 86.026 124.705249) (width 0.15) (layer "F.Cu") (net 25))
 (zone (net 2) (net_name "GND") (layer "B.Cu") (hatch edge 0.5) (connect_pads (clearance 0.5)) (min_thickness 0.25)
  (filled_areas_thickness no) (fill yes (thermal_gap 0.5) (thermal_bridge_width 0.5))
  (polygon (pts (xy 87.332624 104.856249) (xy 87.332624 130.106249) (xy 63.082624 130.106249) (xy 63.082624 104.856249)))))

